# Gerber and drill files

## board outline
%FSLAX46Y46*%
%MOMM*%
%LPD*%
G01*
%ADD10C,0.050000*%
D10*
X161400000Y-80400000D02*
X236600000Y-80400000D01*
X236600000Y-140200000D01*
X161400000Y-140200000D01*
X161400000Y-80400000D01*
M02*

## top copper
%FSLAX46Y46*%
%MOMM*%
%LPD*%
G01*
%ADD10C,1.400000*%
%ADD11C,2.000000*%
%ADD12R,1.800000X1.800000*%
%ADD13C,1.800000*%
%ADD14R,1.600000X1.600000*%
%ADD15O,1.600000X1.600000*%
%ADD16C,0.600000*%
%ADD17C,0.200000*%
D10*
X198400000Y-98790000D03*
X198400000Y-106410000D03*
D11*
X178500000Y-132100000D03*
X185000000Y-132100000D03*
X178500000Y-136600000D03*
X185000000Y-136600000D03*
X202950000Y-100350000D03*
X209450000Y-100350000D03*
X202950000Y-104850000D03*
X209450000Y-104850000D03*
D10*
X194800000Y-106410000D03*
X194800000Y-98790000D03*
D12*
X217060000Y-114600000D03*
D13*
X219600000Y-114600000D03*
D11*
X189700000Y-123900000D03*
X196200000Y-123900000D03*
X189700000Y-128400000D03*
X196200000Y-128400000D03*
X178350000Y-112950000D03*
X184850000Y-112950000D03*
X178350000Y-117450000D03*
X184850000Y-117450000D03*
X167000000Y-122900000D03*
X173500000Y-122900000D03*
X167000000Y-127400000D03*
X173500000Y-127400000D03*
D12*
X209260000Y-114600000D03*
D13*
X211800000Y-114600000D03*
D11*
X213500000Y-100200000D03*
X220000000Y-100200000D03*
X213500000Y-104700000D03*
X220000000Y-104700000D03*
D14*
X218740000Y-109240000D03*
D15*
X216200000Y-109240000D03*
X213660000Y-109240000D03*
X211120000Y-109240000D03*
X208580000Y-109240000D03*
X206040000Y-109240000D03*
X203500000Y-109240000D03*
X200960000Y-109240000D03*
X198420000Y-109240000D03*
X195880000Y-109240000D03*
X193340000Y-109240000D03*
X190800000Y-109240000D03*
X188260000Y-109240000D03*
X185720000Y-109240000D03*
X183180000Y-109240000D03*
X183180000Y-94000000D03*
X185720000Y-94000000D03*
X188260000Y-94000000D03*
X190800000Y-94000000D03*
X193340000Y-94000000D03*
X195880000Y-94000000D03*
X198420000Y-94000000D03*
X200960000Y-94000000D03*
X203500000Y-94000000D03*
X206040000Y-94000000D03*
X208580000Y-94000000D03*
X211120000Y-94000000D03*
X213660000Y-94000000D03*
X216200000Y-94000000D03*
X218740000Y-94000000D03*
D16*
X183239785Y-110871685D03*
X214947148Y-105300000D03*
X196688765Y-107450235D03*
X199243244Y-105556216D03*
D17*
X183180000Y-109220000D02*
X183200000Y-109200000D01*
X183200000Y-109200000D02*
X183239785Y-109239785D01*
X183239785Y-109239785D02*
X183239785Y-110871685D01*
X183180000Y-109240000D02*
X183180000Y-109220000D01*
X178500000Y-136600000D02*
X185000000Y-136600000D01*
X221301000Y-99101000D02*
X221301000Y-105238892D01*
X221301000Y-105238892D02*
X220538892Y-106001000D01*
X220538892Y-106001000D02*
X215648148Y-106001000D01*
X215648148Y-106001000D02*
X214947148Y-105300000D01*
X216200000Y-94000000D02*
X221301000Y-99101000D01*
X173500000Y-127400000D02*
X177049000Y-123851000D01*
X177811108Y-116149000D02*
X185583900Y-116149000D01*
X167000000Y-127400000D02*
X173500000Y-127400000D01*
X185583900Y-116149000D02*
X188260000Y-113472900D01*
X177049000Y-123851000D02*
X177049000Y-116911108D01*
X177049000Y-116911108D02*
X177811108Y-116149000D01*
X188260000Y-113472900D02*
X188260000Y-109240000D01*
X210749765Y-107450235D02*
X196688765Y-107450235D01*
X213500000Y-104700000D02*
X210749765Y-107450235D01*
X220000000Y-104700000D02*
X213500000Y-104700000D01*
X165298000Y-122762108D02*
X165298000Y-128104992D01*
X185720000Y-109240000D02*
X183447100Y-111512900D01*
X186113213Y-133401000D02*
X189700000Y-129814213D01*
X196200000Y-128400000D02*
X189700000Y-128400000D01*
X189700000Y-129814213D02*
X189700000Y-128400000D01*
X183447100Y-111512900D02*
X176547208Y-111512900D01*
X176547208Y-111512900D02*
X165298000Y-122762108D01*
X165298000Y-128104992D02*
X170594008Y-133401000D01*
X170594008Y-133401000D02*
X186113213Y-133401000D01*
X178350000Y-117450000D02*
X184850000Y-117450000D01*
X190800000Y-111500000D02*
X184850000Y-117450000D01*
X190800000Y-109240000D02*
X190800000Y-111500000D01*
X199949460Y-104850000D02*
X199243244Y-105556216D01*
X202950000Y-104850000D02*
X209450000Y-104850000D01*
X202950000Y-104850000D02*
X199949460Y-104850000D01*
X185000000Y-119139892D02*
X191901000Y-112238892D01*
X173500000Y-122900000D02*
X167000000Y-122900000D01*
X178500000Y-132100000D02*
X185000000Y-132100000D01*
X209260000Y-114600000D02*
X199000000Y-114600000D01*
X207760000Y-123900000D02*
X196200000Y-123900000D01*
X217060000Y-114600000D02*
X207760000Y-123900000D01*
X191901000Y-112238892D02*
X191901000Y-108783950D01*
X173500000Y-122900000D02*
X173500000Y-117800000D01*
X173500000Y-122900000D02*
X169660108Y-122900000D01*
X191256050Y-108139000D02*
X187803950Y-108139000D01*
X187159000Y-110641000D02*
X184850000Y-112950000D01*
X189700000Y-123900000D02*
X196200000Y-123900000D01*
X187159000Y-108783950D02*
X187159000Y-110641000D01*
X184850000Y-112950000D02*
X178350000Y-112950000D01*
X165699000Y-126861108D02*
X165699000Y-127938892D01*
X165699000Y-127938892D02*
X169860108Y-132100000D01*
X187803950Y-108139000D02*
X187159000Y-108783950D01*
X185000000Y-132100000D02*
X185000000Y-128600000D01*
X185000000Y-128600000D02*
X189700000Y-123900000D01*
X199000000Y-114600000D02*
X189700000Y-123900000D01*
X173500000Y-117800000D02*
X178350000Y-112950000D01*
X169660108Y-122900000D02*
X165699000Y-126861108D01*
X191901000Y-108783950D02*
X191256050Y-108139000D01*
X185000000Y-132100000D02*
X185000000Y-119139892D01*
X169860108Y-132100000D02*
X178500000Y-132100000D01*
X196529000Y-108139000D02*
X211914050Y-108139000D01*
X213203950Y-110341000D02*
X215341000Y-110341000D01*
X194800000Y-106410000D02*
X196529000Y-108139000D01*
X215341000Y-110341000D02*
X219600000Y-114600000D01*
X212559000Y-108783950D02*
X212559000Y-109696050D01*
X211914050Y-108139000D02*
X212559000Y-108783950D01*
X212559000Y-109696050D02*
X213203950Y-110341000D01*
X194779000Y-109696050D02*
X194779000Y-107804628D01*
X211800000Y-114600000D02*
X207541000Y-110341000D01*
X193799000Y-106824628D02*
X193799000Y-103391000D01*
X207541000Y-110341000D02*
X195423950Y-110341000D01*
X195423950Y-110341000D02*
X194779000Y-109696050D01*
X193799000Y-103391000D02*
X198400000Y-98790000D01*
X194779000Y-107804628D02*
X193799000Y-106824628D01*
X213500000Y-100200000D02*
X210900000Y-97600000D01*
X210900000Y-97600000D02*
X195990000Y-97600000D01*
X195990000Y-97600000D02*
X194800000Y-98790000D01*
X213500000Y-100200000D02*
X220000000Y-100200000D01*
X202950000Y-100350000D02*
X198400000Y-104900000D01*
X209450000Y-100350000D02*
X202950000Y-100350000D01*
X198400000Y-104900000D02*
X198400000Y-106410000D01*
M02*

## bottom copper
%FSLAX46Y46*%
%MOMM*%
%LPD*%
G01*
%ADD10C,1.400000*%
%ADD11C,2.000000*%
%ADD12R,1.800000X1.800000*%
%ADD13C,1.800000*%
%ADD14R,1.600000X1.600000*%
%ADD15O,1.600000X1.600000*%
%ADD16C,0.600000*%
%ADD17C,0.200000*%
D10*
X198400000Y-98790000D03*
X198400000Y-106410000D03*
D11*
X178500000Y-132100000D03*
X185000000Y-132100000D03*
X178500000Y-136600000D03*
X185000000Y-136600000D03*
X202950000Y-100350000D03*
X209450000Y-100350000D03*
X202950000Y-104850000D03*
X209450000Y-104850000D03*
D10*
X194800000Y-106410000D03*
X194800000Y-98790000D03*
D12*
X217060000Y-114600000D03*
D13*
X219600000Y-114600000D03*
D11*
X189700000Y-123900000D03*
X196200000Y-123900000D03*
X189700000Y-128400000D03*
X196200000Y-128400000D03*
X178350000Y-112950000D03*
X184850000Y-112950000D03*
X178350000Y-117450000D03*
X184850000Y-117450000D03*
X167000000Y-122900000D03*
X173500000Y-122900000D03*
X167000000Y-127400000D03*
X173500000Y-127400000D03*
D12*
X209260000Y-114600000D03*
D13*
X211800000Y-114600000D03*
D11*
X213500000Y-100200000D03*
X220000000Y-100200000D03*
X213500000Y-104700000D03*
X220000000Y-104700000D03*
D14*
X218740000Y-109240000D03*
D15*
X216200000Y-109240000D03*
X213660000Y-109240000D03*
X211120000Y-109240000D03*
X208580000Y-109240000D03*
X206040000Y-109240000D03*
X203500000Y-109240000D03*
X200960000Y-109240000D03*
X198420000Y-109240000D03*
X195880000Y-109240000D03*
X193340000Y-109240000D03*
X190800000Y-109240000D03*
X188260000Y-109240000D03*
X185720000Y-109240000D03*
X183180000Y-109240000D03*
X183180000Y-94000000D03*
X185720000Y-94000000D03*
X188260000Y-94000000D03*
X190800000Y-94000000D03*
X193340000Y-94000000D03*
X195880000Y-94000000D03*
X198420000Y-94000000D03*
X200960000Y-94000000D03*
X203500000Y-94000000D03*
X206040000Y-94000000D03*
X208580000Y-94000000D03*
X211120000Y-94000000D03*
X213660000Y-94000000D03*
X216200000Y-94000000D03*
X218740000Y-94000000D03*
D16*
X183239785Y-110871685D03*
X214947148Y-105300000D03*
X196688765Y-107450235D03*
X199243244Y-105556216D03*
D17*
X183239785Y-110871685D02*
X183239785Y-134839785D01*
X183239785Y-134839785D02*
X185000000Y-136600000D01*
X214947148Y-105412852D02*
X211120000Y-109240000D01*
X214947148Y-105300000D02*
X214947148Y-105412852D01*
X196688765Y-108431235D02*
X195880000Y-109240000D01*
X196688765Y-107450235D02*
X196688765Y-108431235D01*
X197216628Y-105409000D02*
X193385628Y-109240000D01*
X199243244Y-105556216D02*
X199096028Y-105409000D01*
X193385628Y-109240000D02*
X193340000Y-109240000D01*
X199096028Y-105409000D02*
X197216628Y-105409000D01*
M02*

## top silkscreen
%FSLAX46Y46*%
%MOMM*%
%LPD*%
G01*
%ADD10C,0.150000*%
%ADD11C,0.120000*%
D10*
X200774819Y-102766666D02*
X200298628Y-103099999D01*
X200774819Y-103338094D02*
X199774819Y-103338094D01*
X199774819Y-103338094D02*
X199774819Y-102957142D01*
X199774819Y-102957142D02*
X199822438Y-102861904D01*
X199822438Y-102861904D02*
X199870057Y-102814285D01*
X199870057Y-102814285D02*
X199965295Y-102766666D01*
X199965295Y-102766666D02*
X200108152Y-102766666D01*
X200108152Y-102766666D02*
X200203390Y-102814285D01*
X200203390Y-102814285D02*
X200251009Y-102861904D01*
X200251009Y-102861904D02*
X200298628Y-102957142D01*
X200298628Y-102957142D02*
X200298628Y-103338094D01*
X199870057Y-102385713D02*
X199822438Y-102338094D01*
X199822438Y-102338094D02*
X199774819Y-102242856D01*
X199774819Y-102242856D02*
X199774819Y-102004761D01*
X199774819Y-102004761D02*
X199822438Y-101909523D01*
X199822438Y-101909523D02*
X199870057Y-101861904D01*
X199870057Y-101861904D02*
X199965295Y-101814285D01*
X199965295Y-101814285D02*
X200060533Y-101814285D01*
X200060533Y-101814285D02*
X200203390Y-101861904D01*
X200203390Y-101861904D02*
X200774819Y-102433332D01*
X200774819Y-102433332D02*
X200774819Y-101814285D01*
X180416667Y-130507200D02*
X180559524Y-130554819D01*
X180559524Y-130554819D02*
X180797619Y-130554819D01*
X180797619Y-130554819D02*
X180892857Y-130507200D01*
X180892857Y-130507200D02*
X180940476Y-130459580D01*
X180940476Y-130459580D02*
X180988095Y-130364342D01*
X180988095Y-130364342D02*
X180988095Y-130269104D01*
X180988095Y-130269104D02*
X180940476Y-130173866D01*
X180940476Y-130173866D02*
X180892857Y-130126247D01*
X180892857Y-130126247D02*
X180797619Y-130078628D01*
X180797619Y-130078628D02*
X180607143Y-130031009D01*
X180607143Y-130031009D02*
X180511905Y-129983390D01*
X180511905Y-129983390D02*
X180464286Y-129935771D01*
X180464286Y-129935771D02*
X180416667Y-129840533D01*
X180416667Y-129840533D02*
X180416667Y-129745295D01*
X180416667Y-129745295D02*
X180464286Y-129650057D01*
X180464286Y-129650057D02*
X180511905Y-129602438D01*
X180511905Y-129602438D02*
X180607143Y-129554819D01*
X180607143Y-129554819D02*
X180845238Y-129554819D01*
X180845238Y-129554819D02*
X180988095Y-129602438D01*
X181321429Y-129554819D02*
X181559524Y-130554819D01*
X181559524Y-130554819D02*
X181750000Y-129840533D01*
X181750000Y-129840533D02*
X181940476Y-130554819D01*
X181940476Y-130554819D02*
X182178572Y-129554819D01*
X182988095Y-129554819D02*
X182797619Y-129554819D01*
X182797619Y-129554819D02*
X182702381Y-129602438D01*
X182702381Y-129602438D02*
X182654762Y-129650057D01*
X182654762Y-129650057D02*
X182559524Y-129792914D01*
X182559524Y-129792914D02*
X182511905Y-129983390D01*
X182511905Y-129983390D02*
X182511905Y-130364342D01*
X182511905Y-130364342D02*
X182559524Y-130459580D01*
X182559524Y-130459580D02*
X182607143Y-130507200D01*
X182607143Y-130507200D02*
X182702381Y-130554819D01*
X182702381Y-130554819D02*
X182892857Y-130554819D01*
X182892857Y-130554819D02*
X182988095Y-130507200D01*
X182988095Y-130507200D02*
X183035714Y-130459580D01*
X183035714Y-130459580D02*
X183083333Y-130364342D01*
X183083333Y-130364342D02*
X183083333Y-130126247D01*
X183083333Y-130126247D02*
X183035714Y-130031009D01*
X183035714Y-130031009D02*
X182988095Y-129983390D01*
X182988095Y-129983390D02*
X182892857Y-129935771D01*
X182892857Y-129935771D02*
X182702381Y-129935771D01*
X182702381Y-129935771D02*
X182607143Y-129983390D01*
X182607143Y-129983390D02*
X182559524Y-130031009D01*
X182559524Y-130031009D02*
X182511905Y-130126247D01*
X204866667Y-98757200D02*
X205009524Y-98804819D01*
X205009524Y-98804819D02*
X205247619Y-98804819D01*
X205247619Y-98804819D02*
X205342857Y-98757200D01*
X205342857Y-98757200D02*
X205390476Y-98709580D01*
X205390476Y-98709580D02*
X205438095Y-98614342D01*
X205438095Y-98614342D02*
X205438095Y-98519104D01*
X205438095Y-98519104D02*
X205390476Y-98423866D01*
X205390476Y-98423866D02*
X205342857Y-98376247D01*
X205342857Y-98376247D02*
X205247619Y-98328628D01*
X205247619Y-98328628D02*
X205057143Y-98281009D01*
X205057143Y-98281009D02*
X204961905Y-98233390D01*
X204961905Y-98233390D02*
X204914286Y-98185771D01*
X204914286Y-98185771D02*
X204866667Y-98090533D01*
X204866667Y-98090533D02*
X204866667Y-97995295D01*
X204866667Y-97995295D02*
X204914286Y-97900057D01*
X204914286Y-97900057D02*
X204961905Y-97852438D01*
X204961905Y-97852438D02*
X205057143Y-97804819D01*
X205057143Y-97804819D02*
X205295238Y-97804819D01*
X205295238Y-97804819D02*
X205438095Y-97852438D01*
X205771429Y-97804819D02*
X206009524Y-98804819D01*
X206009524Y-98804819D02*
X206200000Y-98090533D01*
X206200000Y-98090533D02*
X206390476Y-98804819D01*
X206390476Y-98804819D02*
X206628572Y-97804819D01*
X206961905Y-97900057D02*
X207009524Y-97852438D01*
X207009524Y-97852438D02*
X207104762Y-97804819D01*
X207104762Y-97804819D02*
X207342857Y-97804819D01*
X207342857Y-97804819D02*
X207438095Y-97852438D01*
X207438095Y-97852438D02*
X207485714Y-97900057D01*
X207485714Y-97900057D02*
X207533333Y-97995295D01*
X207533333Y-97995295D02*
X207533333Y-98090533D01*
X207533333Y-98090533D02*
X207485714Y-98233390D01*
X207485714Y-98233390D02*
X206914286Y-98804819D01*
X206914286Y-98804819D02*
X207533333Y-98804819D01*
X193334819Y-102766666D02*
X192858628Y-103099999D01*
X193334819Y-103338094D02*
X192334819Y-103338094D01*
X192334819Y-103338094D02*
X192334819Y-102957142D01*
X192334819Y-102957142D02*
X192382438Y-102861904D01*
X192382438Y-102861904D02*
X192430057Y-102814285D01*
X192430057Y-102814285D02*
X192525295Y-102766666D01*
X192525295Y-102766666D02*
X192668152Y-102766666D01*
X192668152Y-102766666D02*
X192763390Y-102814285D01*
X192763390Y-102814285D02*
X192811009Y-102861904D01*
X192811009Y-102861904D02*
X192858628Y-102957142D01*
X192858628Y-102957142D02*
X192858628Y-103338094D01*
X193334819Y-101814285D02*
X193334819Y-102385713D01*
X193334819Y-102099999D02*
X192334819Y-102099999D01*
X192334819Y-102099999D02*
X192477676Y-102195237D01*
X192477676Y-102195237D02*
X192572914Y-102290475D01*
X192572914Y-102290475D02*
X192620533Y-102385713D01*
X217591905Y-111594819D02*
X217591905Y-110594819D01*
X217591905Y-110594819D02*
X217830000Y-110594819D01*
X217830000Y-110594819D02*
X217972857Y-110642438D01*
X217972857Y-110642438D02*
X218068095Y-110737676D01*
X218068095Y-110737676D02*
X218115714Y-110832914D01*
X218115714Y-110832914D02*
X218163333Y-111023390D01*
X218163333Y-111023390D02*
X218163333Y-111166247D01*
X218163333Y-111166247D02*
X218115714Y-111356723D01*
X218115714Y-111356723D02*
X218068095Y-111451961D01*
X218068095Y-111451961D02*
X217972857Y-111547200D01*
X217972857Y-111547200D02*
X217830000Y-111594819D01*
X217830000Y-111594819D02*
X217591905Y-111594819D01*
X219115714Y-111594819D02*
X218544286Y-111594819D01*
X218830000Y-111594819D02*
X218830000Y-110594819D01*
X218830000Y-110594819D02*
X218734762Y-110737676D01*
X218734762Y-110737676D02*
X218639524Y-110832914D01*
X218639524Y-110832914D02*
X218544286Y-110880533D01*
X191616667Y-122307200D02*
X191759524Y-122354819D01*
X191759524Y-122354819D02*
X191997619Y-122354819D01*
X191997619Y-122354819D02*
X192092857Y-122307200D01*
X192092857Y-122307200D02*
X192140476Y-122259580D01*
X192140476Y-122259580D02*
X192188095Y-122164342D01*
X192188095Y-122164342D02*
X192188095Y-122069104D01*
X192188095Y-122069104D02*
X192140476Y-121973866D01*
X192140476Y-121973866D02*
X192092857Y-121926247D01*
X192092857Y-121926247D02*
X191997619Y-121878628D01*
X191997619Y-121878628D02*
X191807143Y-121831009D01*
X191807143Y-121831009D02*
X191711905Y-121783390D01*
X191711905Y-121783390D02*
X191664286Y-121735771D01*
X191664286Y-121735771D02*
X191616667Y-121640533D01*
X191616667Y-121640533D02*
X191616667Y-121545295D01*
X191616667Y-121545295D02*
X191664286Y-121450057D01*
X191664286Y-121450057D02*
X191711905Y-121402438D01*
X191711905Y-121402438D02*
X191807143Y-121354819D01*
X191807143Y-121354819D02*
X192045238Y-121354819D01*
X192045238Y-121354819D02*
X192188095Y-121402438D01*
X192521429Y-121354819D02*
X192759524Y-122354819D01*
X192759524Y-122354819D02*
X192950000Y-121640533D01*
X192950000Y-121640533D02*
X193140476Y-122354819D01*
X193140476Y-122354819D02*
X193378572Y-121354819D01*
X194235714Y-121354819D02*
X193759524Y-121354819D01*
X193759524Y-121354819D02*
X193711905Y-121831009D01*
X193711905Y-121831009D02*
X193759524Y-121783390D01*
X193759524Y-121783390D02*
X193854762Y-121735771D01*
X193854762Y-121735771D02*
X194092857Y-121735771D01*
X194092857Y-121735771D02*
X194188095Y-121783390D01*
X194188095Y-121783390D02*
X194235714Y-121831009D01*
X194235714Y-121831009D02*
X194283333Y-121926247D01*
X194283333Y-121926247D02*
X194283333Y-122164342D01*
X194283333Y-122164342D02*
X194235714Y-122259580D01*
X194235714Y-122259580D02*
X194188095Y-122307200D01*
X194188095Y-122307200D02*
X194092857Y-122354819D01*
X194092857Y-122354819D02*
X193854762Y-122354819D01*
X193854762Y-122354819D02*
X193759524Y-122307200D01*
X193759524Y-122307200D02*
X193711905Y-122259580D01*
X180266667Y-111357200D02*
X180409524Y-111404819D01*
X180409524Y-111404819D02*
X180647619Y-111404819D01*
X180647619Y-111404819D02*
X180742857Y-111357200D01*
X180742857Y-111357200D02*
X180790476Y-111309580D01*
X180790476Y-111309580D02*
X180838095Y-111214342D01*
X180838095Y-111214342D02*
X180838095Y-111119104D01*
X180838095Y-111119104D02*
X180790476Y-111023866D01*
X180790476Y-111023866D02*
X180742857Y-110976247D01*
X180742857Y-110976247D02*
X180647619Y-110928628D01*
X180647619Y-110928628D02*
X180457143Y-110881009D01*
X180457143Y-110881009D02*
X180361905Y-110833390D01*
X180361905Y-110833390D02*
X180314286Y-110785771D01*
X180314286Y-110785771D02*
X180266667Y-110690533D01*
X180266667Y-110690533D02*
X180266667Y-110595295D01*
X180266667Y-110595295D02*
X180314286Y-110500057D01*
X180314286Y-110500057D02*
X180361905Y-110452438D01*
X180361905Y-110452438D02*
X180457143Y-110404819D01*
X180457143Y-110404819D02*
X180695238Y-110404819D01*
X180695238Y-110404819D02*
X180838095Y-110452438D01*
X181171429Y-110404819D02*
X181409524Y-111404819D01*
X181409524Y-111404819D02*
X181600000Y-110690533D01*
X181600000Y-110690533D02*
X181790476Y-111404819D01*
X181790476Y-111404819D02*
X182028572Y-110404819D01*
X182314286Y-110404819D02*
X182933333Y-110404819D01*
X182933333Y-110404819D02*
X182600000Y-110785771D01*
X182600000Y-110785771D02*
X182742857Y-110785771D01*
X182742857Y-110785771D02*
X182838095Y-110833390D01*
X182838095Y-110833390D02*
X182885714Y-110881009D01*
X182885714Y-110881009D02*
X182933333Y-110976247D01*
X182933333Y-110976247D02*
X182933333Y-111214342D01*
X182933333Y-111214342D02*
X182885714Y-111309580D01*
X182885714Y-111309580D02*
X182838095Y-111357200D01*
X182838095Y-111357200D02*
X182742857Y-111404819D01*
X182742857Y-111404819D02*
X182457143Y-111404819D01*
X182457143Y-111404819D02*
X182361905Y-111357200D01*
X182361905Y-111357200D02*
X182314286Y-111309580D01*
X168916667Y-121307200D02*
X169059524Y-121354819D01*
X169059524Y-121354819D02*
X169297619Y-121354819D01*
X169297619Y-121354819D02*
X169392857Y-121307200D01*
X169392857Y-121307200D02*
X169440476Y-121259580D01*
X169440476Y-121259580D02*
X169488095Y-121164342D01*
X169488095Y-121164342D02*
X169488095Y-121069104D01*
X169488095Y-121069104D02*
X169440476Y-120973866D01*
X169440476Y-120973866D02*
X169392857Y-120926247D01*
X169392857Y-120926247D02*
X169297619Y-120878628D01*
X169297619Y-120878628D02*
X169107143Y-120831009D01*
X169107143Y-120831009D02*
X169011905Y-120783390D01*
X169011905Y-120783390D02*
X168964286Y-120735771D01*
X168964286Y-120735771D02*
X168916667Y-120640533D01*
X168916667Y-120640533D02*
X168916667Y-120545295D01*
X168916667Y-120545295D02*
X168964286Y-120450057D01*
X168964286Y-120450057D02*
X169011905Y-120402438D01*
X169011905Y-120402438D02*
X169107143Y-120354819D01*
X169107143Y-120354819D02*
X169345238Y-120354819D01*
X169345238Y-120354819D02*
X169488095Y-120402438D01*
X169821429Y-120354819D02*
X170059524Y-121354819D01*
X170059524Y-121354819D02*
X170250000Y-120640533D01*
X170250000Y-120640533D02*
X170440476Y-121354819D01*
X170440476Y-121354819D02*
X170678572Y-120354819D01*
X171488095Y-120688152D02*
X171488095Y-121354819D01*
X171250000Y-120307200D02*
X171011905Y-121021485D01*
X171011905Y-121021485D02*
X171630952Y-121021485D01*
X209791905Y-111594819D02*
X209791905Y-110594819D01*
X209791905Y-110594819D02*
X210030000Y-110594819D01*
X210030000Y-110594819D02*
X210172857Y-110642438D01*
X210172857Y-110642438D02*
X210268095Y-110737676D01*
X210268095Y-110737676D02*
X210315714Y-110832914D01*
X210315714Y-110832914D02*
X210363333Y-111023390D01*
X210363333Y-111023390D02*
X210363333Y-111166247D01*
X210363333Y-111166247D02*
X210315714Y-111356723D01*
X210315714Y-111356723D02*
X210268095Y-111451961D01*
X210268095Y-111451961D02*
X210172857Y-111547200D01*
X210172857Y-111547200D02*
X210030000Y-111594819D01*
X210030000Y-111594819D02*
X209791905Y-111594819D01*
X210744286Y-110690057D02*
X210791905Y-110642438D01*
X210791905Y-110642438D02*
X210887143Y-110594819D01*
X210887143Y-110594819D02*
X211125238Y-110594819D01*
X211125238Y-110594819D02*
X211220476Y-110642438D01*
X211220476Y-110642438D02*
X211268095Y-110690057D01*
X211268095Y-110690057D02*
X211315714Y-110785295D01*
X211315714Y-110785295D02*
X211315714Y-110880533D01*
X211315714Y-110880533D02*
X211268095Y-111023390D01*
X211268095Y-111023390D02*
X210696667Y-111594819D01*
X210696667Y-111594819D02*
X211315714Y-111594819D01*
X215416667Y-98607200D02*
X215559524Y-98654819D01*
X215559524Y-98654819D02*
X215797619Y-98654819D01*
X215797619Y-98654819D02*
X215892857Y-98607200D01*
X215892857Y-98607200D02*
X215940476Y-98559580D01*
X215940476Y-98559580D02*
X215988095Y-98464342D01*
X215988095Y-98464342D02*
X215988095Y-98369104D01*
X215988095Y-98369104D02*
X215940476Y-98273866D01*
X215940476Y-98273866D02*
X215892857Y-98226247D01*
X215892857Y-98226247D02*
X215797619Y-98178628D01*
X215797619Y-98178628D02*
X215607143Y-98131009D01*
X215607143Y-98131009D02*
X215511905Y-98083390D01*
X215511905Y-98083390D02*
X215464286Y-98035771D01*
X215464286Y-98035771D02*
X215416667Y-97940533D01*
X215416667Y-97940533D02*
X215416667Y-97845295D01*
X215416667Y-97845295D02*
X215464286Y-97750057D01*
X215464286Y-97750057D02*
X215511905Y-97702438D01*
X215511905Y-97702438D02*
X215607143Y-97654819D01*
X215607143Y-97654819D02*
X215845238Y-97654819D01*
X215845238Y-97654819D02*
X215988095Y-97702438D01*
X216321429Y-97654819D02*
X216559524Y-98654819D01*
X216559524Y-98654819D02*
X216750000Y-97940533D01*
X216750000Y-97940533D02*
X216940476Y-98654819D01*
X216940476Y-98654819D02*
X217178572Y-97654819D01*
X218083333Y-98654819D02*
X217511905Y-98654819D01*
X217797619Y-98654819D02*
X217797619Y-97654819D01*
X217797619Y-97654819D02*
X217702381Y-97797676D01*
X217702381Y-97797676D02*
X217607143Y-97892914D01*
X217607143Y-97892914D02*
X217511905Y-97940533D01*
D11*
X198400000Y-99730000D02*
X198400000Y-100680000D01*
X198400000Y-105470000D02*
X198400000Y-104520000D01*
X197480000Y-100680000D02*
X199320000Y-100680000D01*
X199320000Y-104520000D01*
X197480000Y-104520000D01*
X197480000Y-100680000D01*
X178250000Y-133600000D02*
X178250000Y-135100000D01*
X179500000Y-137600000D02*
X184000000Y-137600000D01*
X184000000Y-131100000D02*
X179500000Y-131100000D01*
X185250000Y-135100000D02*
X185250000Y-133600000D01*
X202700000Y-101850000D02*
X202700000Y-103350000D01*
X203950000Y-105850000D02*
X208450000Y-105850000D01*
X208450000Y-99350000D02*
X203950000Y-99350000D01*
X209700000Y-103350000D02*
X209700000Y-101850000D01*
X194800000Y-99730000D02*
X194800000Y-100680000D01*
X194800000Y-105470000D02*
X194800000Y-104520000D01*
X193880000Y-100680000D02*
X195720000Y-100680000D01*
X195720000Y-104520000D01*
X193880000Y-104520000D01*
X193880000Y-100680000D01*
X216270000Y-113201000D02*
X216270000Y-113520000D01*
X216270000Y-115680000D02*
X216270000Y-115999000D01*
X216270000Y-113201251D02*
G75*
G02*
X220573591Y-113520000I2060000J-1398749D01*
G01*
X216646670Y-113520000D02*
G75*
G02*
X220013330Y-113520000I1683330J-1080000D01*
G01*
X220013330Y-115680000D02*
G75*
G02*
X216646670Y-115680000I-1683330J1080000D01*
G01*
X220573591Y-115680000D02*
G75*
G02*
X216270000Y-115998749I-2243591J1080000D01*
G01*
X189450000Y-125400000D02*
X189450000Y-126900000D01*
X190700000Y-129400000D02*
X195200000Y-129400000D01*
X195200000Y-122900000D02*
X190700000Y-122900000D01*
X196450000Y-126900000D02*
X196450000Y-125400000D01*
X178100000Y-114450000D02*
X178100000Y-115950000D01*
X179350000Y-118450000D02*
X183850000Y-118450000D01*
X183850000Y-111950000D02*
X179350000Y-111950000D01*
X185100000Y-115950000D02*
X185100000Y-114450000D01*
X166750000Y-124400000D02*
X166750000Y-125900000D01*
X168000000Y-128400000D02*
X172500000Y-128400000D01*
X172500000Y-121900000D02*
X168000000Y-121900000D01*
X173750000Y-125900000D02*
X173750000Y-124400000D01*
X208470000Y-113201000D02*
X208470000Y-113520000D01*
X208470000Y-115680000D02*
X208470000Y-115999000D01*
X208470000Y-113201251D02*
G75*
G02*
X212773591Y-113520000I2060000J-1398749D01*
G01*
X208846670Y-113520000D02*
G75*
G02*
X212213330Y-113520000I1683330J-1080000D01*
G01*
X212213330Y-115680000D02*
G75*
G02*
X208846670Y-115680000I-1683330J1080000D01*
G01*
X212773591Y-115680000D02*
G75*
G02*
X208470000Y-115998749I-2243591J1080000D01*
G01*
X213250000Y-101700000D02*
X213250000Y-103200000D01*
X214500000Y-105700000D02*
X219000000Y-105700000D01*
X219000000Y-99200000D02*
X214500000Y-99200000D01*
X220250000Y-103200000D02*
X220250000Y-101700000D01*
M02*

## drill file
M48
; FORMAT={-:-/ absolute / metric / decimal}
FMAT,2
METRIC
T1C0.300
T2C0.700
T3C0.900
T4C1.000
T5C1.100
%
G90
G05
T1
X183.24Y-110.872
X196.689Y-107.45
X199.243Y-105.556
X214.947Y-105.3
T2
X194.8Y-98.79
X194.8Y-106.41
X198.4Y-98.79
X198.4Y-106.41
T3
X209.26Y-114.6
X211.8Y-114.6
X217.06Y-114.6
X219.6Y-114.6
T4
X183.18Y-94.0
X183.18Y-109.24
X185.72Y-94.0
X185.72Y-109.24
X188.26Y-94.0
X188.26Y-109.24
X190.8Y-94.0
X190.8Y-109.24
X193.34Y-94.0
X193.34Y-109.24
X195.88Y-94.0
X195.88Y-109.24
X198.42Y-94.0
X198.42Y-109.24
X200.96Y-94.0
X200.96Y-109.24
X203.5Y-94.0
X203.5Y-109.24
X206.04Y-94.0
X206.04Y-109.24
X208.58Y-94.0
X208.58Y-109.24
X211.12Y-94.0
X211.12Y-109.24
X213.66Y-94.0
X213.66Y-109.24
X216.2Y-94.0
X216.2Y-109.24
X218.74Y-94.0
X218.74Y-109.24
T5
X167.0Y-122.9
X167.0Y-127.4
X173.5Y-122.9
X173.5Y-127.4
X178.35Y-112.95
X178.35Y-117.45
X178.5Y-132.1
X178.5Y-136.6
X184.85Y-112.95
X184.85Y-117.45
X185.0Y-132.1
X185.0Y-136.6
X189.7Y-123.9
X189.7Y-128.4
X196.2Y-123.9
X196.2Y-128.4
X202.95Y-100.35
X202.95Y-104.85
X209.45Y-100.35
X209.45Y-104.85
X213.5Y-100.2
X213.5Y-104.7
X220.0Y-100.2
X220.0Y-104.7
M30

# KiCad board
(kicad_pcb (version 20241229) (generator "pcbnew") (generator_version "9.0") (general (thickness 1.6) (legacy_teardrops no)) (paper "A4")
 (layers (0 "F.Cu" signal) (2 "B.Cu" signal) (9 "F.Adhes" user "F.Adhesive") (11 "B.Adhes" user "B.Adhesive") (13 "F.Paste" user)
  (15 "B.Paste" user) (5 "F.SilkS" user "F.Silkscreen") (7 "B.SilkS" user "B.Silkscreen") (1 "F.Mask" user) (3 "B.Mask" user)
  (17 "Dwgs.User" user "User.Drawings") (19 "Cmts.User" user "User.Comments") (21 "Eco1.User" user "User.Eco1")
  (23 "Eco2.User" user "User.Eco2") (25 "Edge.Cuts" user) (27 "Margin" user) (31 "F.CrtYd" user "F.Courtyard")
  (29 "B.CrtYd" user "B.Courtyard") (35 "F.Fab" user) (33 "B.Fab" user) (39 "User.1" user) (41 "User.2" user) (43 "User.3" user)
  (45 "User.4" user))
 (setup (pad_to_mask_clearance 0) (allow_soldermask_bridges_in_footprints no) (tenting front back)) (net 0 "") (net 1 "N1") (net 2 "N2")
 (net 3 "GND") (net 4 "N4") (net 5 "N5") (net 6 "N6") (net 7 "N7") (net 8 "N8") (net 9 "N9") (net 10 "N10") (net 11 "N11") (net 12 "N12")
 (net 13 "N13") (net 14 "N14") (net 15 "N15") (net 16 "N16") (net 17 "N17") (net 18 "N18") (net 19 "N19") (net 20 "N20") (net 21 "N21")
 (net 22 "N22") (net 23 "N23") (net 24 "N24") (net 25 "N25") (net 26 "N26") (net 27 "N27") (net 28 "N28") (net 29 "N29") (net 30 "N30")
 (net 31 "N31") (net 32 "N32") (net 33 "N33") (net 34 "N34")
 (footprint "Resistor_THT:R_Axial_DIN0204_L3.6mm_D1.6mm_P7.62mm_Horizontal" (layer "F.Cu") (at 198.4 98.79 -90)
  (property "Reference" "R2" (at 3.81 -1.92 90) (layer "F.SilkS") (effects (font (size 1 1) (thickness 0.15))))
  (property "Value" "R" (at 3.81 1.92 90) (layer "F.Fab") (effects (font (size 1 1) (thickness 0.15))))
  (fp_line (start 0.94 0) (end 1.89 0) (stroke (width 0.12) (type solid)) (layer "F.SilkS"))
  (fp_line (start 6.68 0) (end 5.73 0) (stroke (width 0.12) (type solid)) (layer "F.SilkS"))
  (fp_rect (start 1.89 -0.92) (end 5.73 0.92) (stroke (width 0.12) (type solid)) (fill no) (layer "F.SilkS"))
  (pad "1" thru_hole circle (at 0 0 270) (size 1.4 1.4) (drill 0.7) (layers "*.Cu" "*.Mask") (remove_unused_layers no) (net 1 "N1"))
  (pad "2" thru_hole circle (at 7.62 0 270) (size 1.4 1.4) (drill 0.7) (layers "*.Cu" "*.Mask") (remove_unused_layers no) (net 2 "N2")))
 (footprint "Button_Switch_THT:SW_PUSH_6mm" (layer "F.Cu") (at 178.5 132.1)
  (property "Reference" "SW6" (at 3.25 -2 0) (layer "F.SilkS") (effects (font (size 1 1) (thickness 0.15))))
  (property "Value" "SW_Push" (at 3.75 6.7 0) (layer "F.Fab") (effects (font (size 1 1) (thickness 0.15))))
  (fp_line (start -0.25 1.5) (end -0.25 3) (stroke (width 0.12) (type solid)) (layer "F.SilkS"))
  (fp_line (start 1 5.5) (end 5.5 5.5) (stroke (width 0.12) (type solid)) (layer "F.SilkS"))
  (fp_line (start 5.5 -1) (end 1 -1) (stroke (width 0.12) (type solid)) (layer "F.SilkS"))
  (fp_line (start 6.75 3) (end 6.75 1.5) (stroke (width 0.12) (type solid)) (layer "F.SilkS"))
  (pad "1" thru_hole circle (at 0 0 90) (size 2 2) (drill 1.1) (layers "*.Cu" "*.Mask") (remove_unused_layers no) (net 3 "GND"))
  (pad "1" thru_hole circle (at 6.5 0 90) (size 2 2) (drill 1.1) (layers "*.Cu" "*.Mask") (remove_unused_layers no) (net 3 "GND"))
  (pad "2" thru_hole circle (at 0 4.5 90) (size 2 2) (drill 1.1) (layers "*.Cu" "*.Mask") (remove_unused_layers no) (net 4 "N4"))
  (pad "2" thru_hole circle (at 6.5 4.5 90) (size 2 2) (drill 1.1) (layers "*.Cu" "*.Mask") (remove_unused_layers no) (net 4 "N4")))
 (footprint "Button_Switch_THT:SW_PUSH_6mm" (layer "F.Cu") (at 202.95 100.35)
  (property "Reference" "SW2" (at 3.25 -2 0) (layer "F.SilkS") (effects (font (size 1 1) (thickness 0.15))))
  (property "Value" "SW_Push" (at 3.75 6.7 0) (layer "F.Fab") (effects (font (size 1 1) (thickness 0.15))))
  (fp_line (start -0.25 1.5) (end -0.25 3) (stroke (width 0.12) (type solid)) (layer "F.SilkS"))
  (fp_line (start 1 5.5) (end 5.5 5.5) (stroke (width 0.12) (type solid)) (layer "F.SilkS"))
  (fp_line (start 5.5 -1) (end 1 -1) (stroke (width 0.12) (type solid)) (layer "F.SilkS"))
  (fp_line (start 6.75 3) (end 6.75 1.5) (stroke (width 0.12) (type solid)) (layer "F.SilkS"))
  (pad "1" thru_hole circle (at 0 0 90) (size 2 2) (drill 1.1) (layers "*.Cu" "*.Mask") (remove_unused_layers no) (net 2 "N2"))
  (pad "1" thru_hole circle (at 6.5 0 90) (size 2 2) (drill 1.1) (layers "*.Cu" "*.Mask") (remove_unused_layers no) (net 2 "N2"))
  (pad "2" thru_hole circle (at 0 4.5 90) (size 2 2) (drill 1.1) (layers "*.Cu" "*.Mask") (remove_unused_layers no) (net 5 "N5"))
  (pad "2" thru_hole circle (at 6.5 4.5 90) (size 2 2) (drill 1.1) (layers "*.Cu" "*.Mask") (remove_unused_layers no) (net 5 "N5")))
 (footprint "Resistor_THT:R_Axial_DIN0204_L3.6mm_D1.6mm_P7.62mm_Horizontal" (layer "F.Cu") (at 194.8 106.41 90)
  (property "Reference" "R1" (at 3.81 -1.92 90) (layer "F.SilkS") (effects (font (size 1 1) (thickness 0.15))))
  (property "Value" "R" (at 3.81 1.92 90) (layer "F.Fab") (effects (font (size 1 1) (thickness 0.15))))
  (fp_line (start 6.68 0) (end 5.73 0) (stroke (width 0.12) (type solid)) (layer "F.SilkS"))
  (fp_line (start 0.94 0) (end 1.89 0) (stroke (width 0.12) (type solid)) (layer "F.SilkS"))
  (fp_rect (start 1.89 -0.92) (end 5.73 0.92) (stroke (width 0.12) (type solid)) (fill no) (layer "F.SilkS"))
  (pad "1" thru_hole circle (at 0 0 90) (size 1.4 1.4) (drill 0.7) (layers "*.Cu" "*.Mask") (remove_unused_layers no) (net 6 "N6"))
  (pad "2" thru_hole circle (at 7.62 0 90) (size 1.4 1.4) (drill 0.7) (layers "*.Cu" "*.Mask") (remove_unused_layers no) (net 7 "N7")))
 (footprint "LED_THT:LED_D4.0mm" (layer "F.Cu") (at 217.06 114.6)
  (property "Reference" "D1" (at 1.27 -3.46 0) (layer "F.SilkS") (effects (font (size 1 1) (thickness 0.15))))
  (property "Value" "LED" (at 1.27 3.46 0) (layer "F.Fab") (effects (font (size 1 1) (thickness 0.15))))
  (fp_line (start -0.79 -1.399) (end -0.79 -1.08) (stroke (width 0.12) (type solid)) (layer "F.SilkS"))
  (fp_line (start -0.79 1.08) (end -0.79 1.399) (stroke (width 0.12) (type solid)) (layer "F.SilkS"))
  (fp_arc (start -0.79 -1.398749) (mid 1.45392 -2.483198) (end 3.513591 -1.08) (stroke (width 0.12) (type solid)) (layer "F.SilkS"))
  (fp_arc (start -0.41333 -1.08) (mid 1.27 -2) (end 2.95333 -1.08) (stroke (width 0.12) (type solid)) (layer "F.SilkS"))
  (fp_arc (start 2.95333 1.08) (mid 1.27 2) (end -0.41333 1.08) (stroke (width 0.12) (type solid)) (layer "F.SilkS"))
  (fp_arc (start 3.513591 1.08) (mid 1.45392 2.483198) (end -0.79 1.398749) (stroke (width 0.12) (type solid)) (layer "F.SilkS"))
  (pad "1" thru_hole rect (at 0 0) (size 1.8 1.8) (drill 0.9) (layers "*.Cu" "*.Mask") (remove_unused_layers no) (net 3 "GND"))
  (pad "2" thru_hole circle (at 2.54 0) (size 1.8 1.8) (drill 0.9) (layers "*.Cu" "*.Mask") (remove_unused_layers no) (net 6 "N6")))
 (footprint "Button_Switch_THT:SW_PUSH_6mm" (layer "F.Cu") (at 189.7 123.9)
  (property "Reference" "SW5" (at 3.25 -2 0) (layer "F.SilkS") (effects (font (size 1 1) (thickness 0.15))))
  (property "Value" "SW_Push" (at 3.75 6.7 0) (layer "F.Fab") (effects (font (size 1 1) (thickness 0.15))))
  (fp_line (start -0.25 1.5) (end -0.25 3) (stroke (width 0.12) (type solid)) (layer "F.SilkS"))
  (fp_line (start 1 5.5) (end 5.5 5.5) (stroke (width 0.12) (type solid)) (layer "F.SilkS"))
  (fp_line (start 5.5 -1) (end 1 -1) (stroke (width 0.12) (type solid)) (layer "F.SilkS"))
  (fp_line (start 6.75 3) (end 6.75 1.5) (stroke (width 0.12) (type solid)) (layer "F.SilkS"))
  (pad "1" thru_hole circle (at 0 0 90) (size 2 2) (drill 1.1) (layers "*.Cu" "*.Mask") (remove_unused_layers no) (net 3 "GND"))
  (pad "1" thru_hole circle (at 6.5 0 90) (size 2 2) (drill 1.1) (layers "*.Cu" "*.Mask") (remove_unused_layers no) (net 3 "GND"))
  (pad "2" thru_hole circle (at 0 4.5 90) (size 2 2) (drill 1.1) (layers "*.Cu" "*.Mask") (remove_unused_layers no) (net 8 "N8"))
  (pad "2" thru_hole circle (at 6.5 4.5 90) (size 2 2) (drill 1.1) (layers "*.Cu" "*.Mask") (remove_unused_layers no) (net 8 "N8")))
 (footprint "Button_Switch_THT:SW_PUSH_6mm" (layer "F.Cu") (at 178.35 112.95)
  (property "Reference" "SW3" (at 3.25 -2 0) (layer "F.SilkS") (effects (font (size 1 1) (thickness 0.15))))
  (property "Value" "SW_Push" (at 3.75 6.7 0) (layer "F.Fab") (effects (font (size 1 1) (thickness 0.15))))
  (fp_line (start -0.25 1.5) (end -0.25 3) (stroke (width 0.12) (type solid)) (layer "F.SilkS"))
  (fp_line (start 1 5.5) (end 5.5 5.5) (stroke (width 0.12) (type solid)) (layer "F.SilkS"))
  (fp_line (start 5.5 -1) (end 1 -1) (stroke (width 0.12) (type solid)) (layer "F.SilkS"))
  (fp_line (start 6.75 3) (end 6.75 1.5) (stroke (width 0.12) (type solid)) (layer "F.SilkS"))
  (pad "1" thru_hole circle (at 0 0 90) (size 2 2) (drill 1.1) (layers "*.Cu" "*.Mask") (remove_unused_layers no) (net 3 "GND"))
  (pad "1" thru_hole circle (at 6.5 0 90) (size 2 2) (drill 1.1) (layers "*.Cu" "*.Mask") (remove_unused_layers no) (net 3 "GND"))
  (pad "2" thru_hole circle (at 0 4.5 90) (size 2 2) (drill 1.1) (layers "*.Cu" "*.Mask") (remove_unused_layers no) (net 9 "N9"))
  (pad "2" thru_hole circle (at 6.5 4.5 90) (size 2 2) (drill 1.1) (layers "*.Cu" "*.Mask") (remove_unused_layers no) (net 9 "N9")))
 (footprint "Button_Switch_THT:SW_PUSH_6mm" (layer "F.Cu") (at 167 122.9)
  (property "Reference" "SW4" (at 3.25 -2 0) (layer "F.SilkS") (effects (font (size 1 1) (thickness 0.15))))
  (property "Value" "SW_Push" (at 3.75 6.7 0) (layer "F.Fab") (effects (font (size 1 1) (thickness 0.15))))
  (fp_line (start -0.25 1.5) (end -0.25 3) (stroke (width 0.12) (type solid)) (layer "F.SilkS"))
  (fp_line (start 1 5.5) (end 5.5 5.5) (stroke (width 0.12) (type solid)) (layer "F.SilkS"))
  (fp_line (start 5.5 -1) (end 1 -1) (stroke (width 0.12) (type solid)) (layer "F.SilkS"))
  (fp_line (start 6.75 3) (end 6.75 1.5) (stroke (width 0.12) (type solid)) (layer "F.SilkS"))
  (pad "1" thru_hole circle (at 0 0 90) (size 2 2) (drill 1.1) (layers "*.Cu" "*.Mask") (remove_unused_layers no) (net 3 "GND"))
  (pad "1" thru_hole circle (at 6.5 0 90) (size 2 2) (drill 1.1) (layers "*.Cu" "*.Mask") (remove_unused_layers no) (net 3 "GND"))
  (pad "2" thru_hole circle (at 0 4.5 90) (size 2 2) (drill 1.1) (layers "*.Cu" "*.Mask") (remove_unused_layers no) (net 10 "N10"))
  (pad "2" thru_hole circle (at 6.5 4.5 90) (size 2 2) (drill 1.1) (layers "*.Cu" "*.Mask") (remove_unused_layers no) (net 10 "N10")))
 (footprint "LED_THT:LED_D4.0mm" (layer "F.Cu") (at 209.26 114.6)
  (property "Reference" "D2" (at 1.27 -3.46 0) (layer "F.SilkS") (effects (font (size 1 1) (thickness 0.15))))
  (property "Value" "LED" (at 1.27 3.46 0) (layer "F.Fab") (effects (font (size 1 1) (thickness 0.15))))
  (fp_line (start -0.79 -1.399) (end -0.79 -1.08) (stroke (width 0.12) (type solid)) (layer "F.SilkS"))
  (fp_line (start -0.79 1.08) (end -0.79 1.399) (stroke (width 0.12) (type solid)) (layer "F.SilkS"))
  (fp_arc (start -0.79 -1.398749) (mid 1.45392 -2.483198) (end 3.513591 -1.08) (stroke (width 0.12) (type solid)) (layer "F.SilkS"))
  (fp_arc (start -0.41333 -1.08) (mid 1.27 -2) (end 2.95333 -1.08) (stroke (width 0.12) (type solid)) (layer "F.SilkS"))
  (fp_arc (start 2.95333 1.08) (mid 1.27 2) (end -0.41333 1.08) (stroke (width 0.12) (type solid)) (layer "F.SilkS"))
  (fp_arc (start 3.513591 1.08) (mid 1.45392 2.483198) (end -0.79 1.398749) (stroke (width 0.12) (type solid)) (layer "F.SilkS"))
  (pad "1" thru_hole rect (at 0 0) (size 1.8 1.8) (drill 0.9) (layers "*.Cu" "*.Mask") (remove_unused_layers no) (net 3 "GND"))
  (pad "2" thru_hole circle (at 2.54 0) (size 1.8 1.8) (drill 0.9) (layers "*.Cu" "*.Mask") (remove_unused_layers no) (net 1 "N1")))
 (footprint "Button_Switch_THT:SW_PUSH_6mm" (layer "F.Cu") (at 213.5 100.2)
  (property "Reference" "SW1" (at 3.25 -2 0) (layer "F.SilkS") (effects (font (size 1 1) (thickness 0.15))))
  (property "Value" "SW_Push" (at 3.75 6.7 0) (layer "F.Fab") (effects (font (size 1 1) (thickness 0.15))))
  (fp_line (start -0.25 1.5) (end -0.25 3) (stroke (width 0.12) (type solid)) (layer "F.SilkS"))
  (fp_line (start 1 5.5) (end 5.5 5.5) (stroke (width 0.12) (type solid)) (layer "F.SilkS"))
  (fp_line (start 5.5 -1) (end 1 -1) (stroke (width 0.12) (type solid)) (layer "F.SilkS"))
  (fp_line (start 6.75 3) (end 6.75 1.5) (stroke (width 0.12) (type solid)) (layer "F.SilkS"))
  (pad "1" thru_hole circle (at 0 0 90) (size 2 2) (drill 1.1) (layers "*.Cu" "*.Mask") (remove_unused_layers no) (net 7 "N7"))
  (pad "1" thru_hole circle (at 6.5 0 90) (size 2 2) (drill 1.1) (layers "*.Cu" "*.Mask") (remove_unused_layers no) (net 7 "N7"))
  (pad "2" thru_hole circle (at 0 4.5 90) (size 2 2) (drill 1.1) (layers "*.Cu" "*.Mask") (remove_unused_layers no) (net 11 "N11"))
  (pad "2" thru_hole circle (at 6.5 4.5 90) (size 2 2) (drill 1.1) (layers "*.Cu" "*.Mask") (remove_unused_layers no) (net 11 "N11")))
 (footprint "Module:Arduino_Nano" (layer "B.Cu") (at 218.74 109.24 90)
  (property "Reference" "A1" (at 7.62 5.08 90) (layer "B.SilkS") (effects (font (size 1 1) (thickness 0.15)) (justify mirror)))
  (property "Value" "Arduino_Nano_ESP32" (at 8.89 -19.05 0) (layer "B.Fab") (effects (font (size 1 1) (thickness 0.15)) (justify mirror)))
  (pad "1" thru_hole rect (at 0 0 90) (size 1.6 1.6) (drill 1) (layers "*.Cu" "*.Mask") (remove_unused_layers no) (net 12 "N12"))
  (pad "2" thru_hole oval (at 0 -2.54 90) (size 1.6 1.6) (drill 1) (layers "*.Cu" "*.Mask") (remove_unused_layers no) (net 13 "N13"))
  (pad "3" thru_hole oval (at 0 -5.08 90) (size 1.6 1.6) (drill 1) (layers "*.Cu" "*.Mask") (remove_unused_layers no) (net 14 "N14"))
  (pad "4" thru_hole oval (at 0 -7.62 90) (size 1.6 1.6) (drill 1) (layers "*.Cu" "*.Mask") (remove_unused_layers no) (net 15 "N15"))
  (pad "5" thru_hole oval (at 0 -10.16 90) (size 1.6 1.6) (drill 1) (layers "*.Cu" "*.Mask") (remove_unused_layers no) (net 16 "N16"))
  (pad "6" thru_hole oval (at 0 -12.7 90) (size 1.6 1.6) (drill 1) (layers "*.Cu" "*.Mask") (remove_unused_layers no) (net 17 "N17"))
  (pad "7" thru_hole oval (at 0 -15.24 90) (size 1.6 1.6) (drill 1) (layers "*.Cu" "*.Mask") (remove_unused_layers no) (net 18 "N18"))
  (pad "8" thru_hole oval (at 0 -17.78 90) (size 1.6 1.6) (drill 1) (layers "*.Cu" "*.Mask") (remove_unused_layers no) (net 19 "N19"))
  (pad "9" thru_hole oval (at 0 -20.32 90) (size 1.6 1.6) (drill 1) (layers "*.Cu" "*.Mask") (remove_unused_layers no) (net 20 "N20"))
  (pad "10" thru_hole oval (at 0 -22.86 90) (size 1.6 1.6) (drill 1) (layers "*.Cu" "*.Mask") (remove_unused_layers no) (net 11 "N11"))
  (pad "11" thru_hole oval (at 0 -25.4 90) (size 1.6 1.6) (drill 1) (layers "*.Cu" "*.Mask") (remove_unused_layers no) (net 5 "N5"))
  (pad "12" thru_hole oval (at 0 -27.94 90) (size 1.6 1.6) (drill 1) (layers "*.Cu" "*.Mask") (remove_unused_layers no) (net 9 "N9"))
  (pad "13" thru_hole oval (at 0 -30.48 90) (size 1.6 1.6) (drill 1) (layers "*.Cu" "*.Mask") (remove_unused_layers no) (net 10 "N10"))
  (pad "14" thru_hole oval (at 0 -33.02 90) (size 1.6 1.6) (drill 1) (layers "*.Cu" "*.Mask") (remove_unused_layers no) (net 8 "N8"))
  (pad "15" thru_hole oval (at 0 -35.56 90) (size 1.6 1.6) (drill 1) (layers "*.Cu" "*.Mask") (remove_unused_layers no) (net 4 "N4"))
  (pad "16" thru_hole oval (at 15.24 -35.56 90) (size 1.6 1.6) (drill 1) (layers "*.Cu" "*.Mask") (remove_unused_layers no) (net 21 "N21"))
  (pad "17" thru_hole oval (at 15.24 -33.02 90) (size 1.6 1.6) (drill 1) (layers "*.Cu" "*.Mask") (remove_unused_layers no) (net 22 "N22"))
  (pad "18" thru_hole oval (at 15.24 -30.48 90) (size 1.6 1.6) (drill 1) (layers "*.Cu" "*.Mask") (remove_unused_layers no) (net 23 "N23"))
  (pad "19" thru_hole oval (at 15.24 -27.94 90) (size 1.6 1.6) (drill 1) (layers "*.Cu" "*.Mask") (remove_unused_layers no) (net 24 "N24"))
  (pad "20" thru_hole oval (at 15.24 -25.4 90) (size 1.6 1.6) (drill 1) (layers "*.Cu" "*.Mask") (remove_unused_layers no) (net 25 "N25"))
  (pad "21" thru_hole oval (at 15.24 -22.86 90) (size 1.6 1.6) (drill 1) (layers "*.Cu" "*.Mask") (remove_unused_layers no) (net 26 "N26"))
  (pad "22" thru_hole oval (at 15.24 -20.32 90) (size 1.6 1.6) (drill 1) (layers "*.Cu" "*.Mask") (remove_unused_layers no) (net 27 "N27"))
  (pad "23" thru_hole oval (at 15.24 -17.78 90) (size 1.6 1.6) (drill 1) (layers "*.Cu" "*.Mask") (remove_unused_layers no) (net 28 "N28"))
  (pad "24" thru_hole oval (at 15.24 -15.24 90) (size 1.6 1.6) (drill 1) (layers "*.Cu" "*.Mask") (remove_unused_layers no) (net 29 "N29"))
  (pad "25" thru_hole oval (at 15.24 -12.7 90) (size 1.6 1.6) (drill 1) (layers "*.Cu" "*.Mask") (remove_unused_layers no) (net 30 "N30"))
  (pad "26" thru_hole oval (at 15.24 -10.16 90) (size 1.6 1.6) (drill 1) (layers "*.Cu" "*.Mask") (remove_unused_layers no) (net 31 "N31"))
  (pad "27" thru_hole oval (at 15.24 -7.62 90) (size 1.6 1.6) (drill 1) (layers "*.Cu" "*.Mask") (remove_unused_layers no) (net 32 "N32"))
  (pad "28" thru_hole oval (at 15.24 -5.08 90) (size 1.6 1.6) (drill 1) (layers "*.Cu" "*.Mask") (remove_unused_layers no) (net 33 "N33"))
  (pad "29" thru_hole oval (at 15.24 -2.54 90) (size 1.6 1.6) (drill 1) (layers "*.Cu" "*.Mask") (remove_unused_layers no) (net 15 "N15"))
  (pad "30" thru_hole oval (at 15.24 0 90) (size 1.6 1.6) (drill 1) (layers "*.Cu" "*.Mask") (remove_unused_layers no) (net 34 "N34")))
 (gr_rect (start 161.4 80.4) (end 236.6 140.2) (stroke (width 0.05) (type default)) (fill no) (layer "Edge.Cuts"))
 (segment (start 183.18 109.22) (end 183.2 109.2) (width 0.2) (layer "F.Cu") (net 4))
 (segment (start 183.2 109.2) (end 183.239785 109.239785) (width 0.2) (layer "F.Cu") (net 4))
 (segment (start 183.239785 109.239785) (end 183.239785 110.871685) (width 0.2) (layer "F.Cu") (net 4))
 (segment (start 183.18 109.24) (end 183.18 109.22) (width 0.2) (layer "F.Cu") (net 4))
 (segment (start 178.5 136.6) (end 185 136.6) (width 0.2) (layer "F.Cu") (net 4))
 (via (at 183.239785 110.871685) (size 0.6) (drill 0.3) (layers "F.Cu" "B.Cu") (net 4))
 (segment (start 183.239785 110.871685) (end 183.239785 134.839785) (width 0.2) (layer "B.Cu") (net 4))
 (segment (start 183.239785 134.839785) (end 185 136.6) (width 0.2) (layer "B.Cu") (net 4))
 (segment (start 221.301 99.101) (end 221.301 105.238892) (width 0.2) (layer "F.Cu") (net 15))
 (segment (start 221.301 105.238892) (end 220.538892 106.001) (width 0.2) (layer "F.Cu") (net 15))
 (segment (start 220.538892 106.001) (end 215.648148 106.001) (width 0.2) (layer "F.Cu") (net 15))
 (segment (start 215.648148 106.001) (end 214.947148 105.3) (width 0.2) (layer "F.Cu") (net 15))
 (segment (start 216.2 94) (end 221.301 99.101) (width 0.2) (layer "F.Cu") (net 15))
 (via (at 214.947148 105.3) (size 0.6) (drill 0.3) (layers "F.Cu" "B.Cu") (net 15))
 (segment (start 214.947148 105.412852) (end 211.12 109.24) (width 0.2) (layer "B.Cu") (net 15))
 (segment (start 214.947148 105.3) (end 214.947148 105.412852) (width 0.2) (layer "B.Cu") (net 15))
 (segment (start 173.5 127.4) (end 177.049 123.851) (width 0.2) (layer "F.Cu") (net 10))
 (segment (start 177.811108 116.149) (end 185.5839 116.149) (width 0.2) (layer "F.Cu") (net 10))
 (segment (start 167 127.4) (end 173.5 127.4) (width 0.2) (layer "F.Cu") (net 10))
 (segment (start 185.5839 116.149) (end 188.26 113.4729) (width 0.2) (layer "F.Cu") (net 10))
 (segment (start 177.049 123.851) (end 177.049 116.911108) (width 0.2) (layer "F.Cu") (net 10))
 (segment (start 177.049 116.911108) (end 177.811108 116.149) (width 0.2) (layer "F.Cu") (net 10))
 (segment (start 188.26 113.4729) (end 188.26 109.24) (width 0.2) (layer "F.Cu") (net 10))
 (segment (start 210.749765 107.450235) (end 196.688765 107.450235) (width 0.2) (layer "F.Cu") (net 11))
 (segment (start 213.5 104.7) (end 210.749765 107.450235) (width 0.2) (layer "F.Cu") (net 11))
 (segment (start 220 104.7) (end 213.5 104.7) (width 0.2) (layer "F.Cu") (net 11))
 (via (at 196.688765 107.450235) (size 0.6) (drill 0.3) (layers "F.Cu" "B.Cu") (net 11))
 (segment (start 196.688765 108.431235) (end 195.88 109.24) (width 0.2) (layer "B.Cu") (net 11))
 (segment (start 196.688765 107.450235) (end 196.688765 108.431235) (width 0.2) (layer "B.Cu") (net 11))
 (segment (start 165.298 122.762108) (end 165.298 128.104992) (width 0.2) (layer "F.Cu") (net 8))
 (segment (start 185.72 109.24) (end 183.4471 111.5129) (width 0.2) (layer "F.Cu") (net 8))
 (segment (start 186.113213 133.401) (end 189.7 129.814213) (width 0.2) (layer "F.Cu") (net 8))
 (segment (start 196.2 128.4) (end 189.7 128.4) (width 0.2) (layer "F.Cu") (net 8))
 (segment (start 189.7 129.814213) (end 189.7 128.4) (width 0.2) (layer "F.Cu") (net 8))
 (segment (start 183.4471 111.5129) (end 176.547208 111.5129) (width 0.2) (layer "F.Cu") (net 8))
 (segment (start 176.547208 111.5129) (end 165.298 122.762108) (width 0.2) (layer "F.Cu") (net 8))
 (segment (start 165.298 128.104992) (end 170.594008 133.401) (width 0.2) (layer "F.Cu") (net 8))
 (segment (start 170.594008 133.401) (end 186.113213 133.401) (width 0.2) (layer "F.Cu") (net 8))
 (segment (start 178.35 117.45) (end 184.85 117.45) (width 0.2) (layer "F.Cu") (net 9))
 (segment (start 190.8 111.5) (end 184.85 117.45) (width 0.2) (layer "F.Cu") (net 9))
 (segment (start 190.8 109.24) (end 190.8 111.5) (width 0.2) (layer "F.Cu") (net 9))
 (segment (start 199.94946 104.85) (end 199.243244 105.556216) (width 0.2) (layer "F.Cu") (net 5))
 (segment (start 202.95 104.85) (end 209.45 104.85) (width 0.2) (layer "F.Cu") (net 5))
 (segment (start 202.95 104.85) (end 199.94946 104.85) (width 0.2) (layer "F.Cu") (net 5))
 (via (at 199.243244 105.556216) (size 0.6) (drill 0.3) (layers "F.Cu" "B.Cu") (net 5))
 (segment (start 197.216628 105.409) (end 193.385628 109.24) (width 0.2) (layer "B.Cu") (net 5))
 (segment (start 199.243244 105.556216) (end 199.096028 105.409) (width 0.2) (layer "B.Cu") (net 5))
 (segment (start 193.385628 109.24) (end 193.34 109.24) (width 0.2) (layer "B.Cu") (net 5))
 (segment (start 199.096028 105.409) (end 197.216628 105.409) (width 0.2) (layer "B.Cu") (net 5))
 (segment (start 185 119.139892) (end 191.901 112.238892) (width 0.2) (layer "F.Cu") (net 3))
 (segment (start 173.5 122.9) (end 167 122.9) (width 0.2) (layer "F.Cu") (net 3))
 (segment (start 178.5 132.1) (end 185 132.1) (width 0.2) (layer "F.Cu") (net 3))
 (segment (start 209.26 114.6) (end 199 114.6) (width 0.2) (layer "F.Cu") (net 3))
 (segment (start 207.76 123.9) (end 196.2 123.9) (width 0.2) (layer "F.Cu") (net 3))
 (segment (start 217.06 114.6) (end 207.76 123.9) (width 0.2) (layer "F.Cu") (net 3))
 (segment (start 191.901 112.238892) (end 191.901 108.78395) (width 0.2) (layer "F.Cu") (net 3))
 (segment (start 173.5 122.9) (end 173.5 117.8) (width 0.2) (layer "F.Cu") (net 3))
 (segment (start 173.5 122.9) (end 169.660108 122.9) (width 0.2) (layer "F.Cu") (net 3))
 (segment (start 191.25605 108.139) (end 187.80395 108.139) (width 0.2) (layer "F.Cu") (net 3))
 (segment (start 187.159 110.641) (end 184.85 112.95) (width 0.2) (layer "F.Cu") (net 3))
 (segment (start 189.7 123.9) (end 196.2 123.9) (width 0.2) (layer "F.Cu") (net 3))
 (segment (start 187.159 108.78395) (end 187.159 110.641) (width 0.2) (layer "F.Cu") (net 3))
 (segment (start 184.85 112.95) (end 178.35 112.95) (width 0.2) (layer "F.Cu") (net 3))
 (segment (start 165.699 126.861108) (end 165.699 127.938892) (width 0.2) (layer "F.Cu") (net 3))
 (segment (start 165.699 127.938892) (end 169.860108 132.1) (width 0.2) (layer "F.Cu") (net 3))
 (segment (start 187.80395 108.139) (end 187.159 108.78395) (width 0.2) (layer "F.Cu") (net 3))
 (segment (start 185 132.1) (end 185 128.6) (width 0.2) (layer "F.Cu") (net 3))
 (segment (start 185 128.6) (end 189.7 123.9) (width 0.2) (layer "F.Cu") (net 3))
 (segment (start 199 114.6) (end 189.7 123.9) (width 0.2) (layer "F.Cu") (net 3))
 (segment (start 173.5 117.8) (end 178.35 112.95) (width 0.2) (layer "F.Cu") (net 3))
 (segment (start 169.660108 122.9) (end 165.699 126.861108) (width 0.2) (layer "F.Cu") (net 3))
 (segment (start 191.901 108.78395) (end 191.25605 108.139) (width 0.2) (layer "F.Cu") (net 3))
 (segment (start 185 132.1) (end 185 119.139892) (width 0.2) (layer "F.Cu") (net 3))
 (segment (start 169.860108 132.1) (end 178.5 132.1) (width 0.2) (layer "F.Cu") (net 3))
 (segment (start 196.529 108.139) (end 211.91405 108.139) (width 0.2) (layer "F.Cu") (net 6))
 (segment (start 213.20395 110.341) (end 215.341 110.341) (width 0.2) (layer "F.Cu") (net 6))
 (segment (start 194.8 106.41) (end 196.529 108.139) (width 0.2) (layer "F.Cu") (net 6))
 (segment (start 215.341 110.341) (end 219.6 114.6) (width 0.2) (layer "F.Cu") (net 6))
 (segment (start 212.559 108.78395) (end 212.559 109.69605) (width 0.2) (layer "F.Cu") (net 6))
 (segment (start 211.91405 108.139) (end 212.559 108.78395) (width 0.2) (layer "F.Cu") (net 6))
 (segment (start 212.559 109.69605) (end 213.20395 110.341) (width 0.2) (layer "F.Cu") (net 6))
 (segment (start 194.779 109.69605) (end 194.779 107.804628) (width 0.2) (layer "F.Cu") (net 1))
 (segment (start 211.8 114.6) (end 207.541 110.341) (width 0.2) (layer "F.Cu") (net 1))
 (segment (start 193.799 106.824628) (end 193.799 103.391) (width 0.2) (layer "F.Cu") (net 1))
 (segment (start 207.541 110.341) (end 195.42395 110.341) (width 0.2) (layer "F.Cu") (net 1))
 (segment (start 195.42395 110.341) (end 194.779 109.69605) (width 0.2) (layer "F.Cu") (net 1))
 (segment (start 193.799 103.391) (end 198.4 98.79) (width 0.2) (layer "F.Cu") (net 1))
 (segment (start 194.779 107.804628) (end 193.799 106.824628) (width 0.2) (layer "F.Cu") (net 1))
 (segment (start 213.5 100.2) (end 210.9 97.6) (width 0.2) (layer "F.Cu") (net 7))
 (segment (start 210.9 97.6) (end 195.99 97.6) (width 0.2) (layer "F.Cu") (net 7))
 (segment (start 195.99 97.6) (end 194.8 98.79) (width 0.2) (layer "F.Cu") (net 7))
 (segment (start 213.5 100.2) (end 220 100.2) (width 0.2) (layer "F.Cu") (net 7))
 (segment (start 202.95 100.35) (end 198.4 104.9) (width 0.2) (layer "F.Cu") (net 2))
 (segment (start 209.45 100.35) (end 202.95 100.35) (width 0.2) (layer "F.Cu") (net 2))
 (segment (start 198.4 104.9) (end 198.4 106.41) (width 0.2) (layer "F.Cu") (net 2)))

